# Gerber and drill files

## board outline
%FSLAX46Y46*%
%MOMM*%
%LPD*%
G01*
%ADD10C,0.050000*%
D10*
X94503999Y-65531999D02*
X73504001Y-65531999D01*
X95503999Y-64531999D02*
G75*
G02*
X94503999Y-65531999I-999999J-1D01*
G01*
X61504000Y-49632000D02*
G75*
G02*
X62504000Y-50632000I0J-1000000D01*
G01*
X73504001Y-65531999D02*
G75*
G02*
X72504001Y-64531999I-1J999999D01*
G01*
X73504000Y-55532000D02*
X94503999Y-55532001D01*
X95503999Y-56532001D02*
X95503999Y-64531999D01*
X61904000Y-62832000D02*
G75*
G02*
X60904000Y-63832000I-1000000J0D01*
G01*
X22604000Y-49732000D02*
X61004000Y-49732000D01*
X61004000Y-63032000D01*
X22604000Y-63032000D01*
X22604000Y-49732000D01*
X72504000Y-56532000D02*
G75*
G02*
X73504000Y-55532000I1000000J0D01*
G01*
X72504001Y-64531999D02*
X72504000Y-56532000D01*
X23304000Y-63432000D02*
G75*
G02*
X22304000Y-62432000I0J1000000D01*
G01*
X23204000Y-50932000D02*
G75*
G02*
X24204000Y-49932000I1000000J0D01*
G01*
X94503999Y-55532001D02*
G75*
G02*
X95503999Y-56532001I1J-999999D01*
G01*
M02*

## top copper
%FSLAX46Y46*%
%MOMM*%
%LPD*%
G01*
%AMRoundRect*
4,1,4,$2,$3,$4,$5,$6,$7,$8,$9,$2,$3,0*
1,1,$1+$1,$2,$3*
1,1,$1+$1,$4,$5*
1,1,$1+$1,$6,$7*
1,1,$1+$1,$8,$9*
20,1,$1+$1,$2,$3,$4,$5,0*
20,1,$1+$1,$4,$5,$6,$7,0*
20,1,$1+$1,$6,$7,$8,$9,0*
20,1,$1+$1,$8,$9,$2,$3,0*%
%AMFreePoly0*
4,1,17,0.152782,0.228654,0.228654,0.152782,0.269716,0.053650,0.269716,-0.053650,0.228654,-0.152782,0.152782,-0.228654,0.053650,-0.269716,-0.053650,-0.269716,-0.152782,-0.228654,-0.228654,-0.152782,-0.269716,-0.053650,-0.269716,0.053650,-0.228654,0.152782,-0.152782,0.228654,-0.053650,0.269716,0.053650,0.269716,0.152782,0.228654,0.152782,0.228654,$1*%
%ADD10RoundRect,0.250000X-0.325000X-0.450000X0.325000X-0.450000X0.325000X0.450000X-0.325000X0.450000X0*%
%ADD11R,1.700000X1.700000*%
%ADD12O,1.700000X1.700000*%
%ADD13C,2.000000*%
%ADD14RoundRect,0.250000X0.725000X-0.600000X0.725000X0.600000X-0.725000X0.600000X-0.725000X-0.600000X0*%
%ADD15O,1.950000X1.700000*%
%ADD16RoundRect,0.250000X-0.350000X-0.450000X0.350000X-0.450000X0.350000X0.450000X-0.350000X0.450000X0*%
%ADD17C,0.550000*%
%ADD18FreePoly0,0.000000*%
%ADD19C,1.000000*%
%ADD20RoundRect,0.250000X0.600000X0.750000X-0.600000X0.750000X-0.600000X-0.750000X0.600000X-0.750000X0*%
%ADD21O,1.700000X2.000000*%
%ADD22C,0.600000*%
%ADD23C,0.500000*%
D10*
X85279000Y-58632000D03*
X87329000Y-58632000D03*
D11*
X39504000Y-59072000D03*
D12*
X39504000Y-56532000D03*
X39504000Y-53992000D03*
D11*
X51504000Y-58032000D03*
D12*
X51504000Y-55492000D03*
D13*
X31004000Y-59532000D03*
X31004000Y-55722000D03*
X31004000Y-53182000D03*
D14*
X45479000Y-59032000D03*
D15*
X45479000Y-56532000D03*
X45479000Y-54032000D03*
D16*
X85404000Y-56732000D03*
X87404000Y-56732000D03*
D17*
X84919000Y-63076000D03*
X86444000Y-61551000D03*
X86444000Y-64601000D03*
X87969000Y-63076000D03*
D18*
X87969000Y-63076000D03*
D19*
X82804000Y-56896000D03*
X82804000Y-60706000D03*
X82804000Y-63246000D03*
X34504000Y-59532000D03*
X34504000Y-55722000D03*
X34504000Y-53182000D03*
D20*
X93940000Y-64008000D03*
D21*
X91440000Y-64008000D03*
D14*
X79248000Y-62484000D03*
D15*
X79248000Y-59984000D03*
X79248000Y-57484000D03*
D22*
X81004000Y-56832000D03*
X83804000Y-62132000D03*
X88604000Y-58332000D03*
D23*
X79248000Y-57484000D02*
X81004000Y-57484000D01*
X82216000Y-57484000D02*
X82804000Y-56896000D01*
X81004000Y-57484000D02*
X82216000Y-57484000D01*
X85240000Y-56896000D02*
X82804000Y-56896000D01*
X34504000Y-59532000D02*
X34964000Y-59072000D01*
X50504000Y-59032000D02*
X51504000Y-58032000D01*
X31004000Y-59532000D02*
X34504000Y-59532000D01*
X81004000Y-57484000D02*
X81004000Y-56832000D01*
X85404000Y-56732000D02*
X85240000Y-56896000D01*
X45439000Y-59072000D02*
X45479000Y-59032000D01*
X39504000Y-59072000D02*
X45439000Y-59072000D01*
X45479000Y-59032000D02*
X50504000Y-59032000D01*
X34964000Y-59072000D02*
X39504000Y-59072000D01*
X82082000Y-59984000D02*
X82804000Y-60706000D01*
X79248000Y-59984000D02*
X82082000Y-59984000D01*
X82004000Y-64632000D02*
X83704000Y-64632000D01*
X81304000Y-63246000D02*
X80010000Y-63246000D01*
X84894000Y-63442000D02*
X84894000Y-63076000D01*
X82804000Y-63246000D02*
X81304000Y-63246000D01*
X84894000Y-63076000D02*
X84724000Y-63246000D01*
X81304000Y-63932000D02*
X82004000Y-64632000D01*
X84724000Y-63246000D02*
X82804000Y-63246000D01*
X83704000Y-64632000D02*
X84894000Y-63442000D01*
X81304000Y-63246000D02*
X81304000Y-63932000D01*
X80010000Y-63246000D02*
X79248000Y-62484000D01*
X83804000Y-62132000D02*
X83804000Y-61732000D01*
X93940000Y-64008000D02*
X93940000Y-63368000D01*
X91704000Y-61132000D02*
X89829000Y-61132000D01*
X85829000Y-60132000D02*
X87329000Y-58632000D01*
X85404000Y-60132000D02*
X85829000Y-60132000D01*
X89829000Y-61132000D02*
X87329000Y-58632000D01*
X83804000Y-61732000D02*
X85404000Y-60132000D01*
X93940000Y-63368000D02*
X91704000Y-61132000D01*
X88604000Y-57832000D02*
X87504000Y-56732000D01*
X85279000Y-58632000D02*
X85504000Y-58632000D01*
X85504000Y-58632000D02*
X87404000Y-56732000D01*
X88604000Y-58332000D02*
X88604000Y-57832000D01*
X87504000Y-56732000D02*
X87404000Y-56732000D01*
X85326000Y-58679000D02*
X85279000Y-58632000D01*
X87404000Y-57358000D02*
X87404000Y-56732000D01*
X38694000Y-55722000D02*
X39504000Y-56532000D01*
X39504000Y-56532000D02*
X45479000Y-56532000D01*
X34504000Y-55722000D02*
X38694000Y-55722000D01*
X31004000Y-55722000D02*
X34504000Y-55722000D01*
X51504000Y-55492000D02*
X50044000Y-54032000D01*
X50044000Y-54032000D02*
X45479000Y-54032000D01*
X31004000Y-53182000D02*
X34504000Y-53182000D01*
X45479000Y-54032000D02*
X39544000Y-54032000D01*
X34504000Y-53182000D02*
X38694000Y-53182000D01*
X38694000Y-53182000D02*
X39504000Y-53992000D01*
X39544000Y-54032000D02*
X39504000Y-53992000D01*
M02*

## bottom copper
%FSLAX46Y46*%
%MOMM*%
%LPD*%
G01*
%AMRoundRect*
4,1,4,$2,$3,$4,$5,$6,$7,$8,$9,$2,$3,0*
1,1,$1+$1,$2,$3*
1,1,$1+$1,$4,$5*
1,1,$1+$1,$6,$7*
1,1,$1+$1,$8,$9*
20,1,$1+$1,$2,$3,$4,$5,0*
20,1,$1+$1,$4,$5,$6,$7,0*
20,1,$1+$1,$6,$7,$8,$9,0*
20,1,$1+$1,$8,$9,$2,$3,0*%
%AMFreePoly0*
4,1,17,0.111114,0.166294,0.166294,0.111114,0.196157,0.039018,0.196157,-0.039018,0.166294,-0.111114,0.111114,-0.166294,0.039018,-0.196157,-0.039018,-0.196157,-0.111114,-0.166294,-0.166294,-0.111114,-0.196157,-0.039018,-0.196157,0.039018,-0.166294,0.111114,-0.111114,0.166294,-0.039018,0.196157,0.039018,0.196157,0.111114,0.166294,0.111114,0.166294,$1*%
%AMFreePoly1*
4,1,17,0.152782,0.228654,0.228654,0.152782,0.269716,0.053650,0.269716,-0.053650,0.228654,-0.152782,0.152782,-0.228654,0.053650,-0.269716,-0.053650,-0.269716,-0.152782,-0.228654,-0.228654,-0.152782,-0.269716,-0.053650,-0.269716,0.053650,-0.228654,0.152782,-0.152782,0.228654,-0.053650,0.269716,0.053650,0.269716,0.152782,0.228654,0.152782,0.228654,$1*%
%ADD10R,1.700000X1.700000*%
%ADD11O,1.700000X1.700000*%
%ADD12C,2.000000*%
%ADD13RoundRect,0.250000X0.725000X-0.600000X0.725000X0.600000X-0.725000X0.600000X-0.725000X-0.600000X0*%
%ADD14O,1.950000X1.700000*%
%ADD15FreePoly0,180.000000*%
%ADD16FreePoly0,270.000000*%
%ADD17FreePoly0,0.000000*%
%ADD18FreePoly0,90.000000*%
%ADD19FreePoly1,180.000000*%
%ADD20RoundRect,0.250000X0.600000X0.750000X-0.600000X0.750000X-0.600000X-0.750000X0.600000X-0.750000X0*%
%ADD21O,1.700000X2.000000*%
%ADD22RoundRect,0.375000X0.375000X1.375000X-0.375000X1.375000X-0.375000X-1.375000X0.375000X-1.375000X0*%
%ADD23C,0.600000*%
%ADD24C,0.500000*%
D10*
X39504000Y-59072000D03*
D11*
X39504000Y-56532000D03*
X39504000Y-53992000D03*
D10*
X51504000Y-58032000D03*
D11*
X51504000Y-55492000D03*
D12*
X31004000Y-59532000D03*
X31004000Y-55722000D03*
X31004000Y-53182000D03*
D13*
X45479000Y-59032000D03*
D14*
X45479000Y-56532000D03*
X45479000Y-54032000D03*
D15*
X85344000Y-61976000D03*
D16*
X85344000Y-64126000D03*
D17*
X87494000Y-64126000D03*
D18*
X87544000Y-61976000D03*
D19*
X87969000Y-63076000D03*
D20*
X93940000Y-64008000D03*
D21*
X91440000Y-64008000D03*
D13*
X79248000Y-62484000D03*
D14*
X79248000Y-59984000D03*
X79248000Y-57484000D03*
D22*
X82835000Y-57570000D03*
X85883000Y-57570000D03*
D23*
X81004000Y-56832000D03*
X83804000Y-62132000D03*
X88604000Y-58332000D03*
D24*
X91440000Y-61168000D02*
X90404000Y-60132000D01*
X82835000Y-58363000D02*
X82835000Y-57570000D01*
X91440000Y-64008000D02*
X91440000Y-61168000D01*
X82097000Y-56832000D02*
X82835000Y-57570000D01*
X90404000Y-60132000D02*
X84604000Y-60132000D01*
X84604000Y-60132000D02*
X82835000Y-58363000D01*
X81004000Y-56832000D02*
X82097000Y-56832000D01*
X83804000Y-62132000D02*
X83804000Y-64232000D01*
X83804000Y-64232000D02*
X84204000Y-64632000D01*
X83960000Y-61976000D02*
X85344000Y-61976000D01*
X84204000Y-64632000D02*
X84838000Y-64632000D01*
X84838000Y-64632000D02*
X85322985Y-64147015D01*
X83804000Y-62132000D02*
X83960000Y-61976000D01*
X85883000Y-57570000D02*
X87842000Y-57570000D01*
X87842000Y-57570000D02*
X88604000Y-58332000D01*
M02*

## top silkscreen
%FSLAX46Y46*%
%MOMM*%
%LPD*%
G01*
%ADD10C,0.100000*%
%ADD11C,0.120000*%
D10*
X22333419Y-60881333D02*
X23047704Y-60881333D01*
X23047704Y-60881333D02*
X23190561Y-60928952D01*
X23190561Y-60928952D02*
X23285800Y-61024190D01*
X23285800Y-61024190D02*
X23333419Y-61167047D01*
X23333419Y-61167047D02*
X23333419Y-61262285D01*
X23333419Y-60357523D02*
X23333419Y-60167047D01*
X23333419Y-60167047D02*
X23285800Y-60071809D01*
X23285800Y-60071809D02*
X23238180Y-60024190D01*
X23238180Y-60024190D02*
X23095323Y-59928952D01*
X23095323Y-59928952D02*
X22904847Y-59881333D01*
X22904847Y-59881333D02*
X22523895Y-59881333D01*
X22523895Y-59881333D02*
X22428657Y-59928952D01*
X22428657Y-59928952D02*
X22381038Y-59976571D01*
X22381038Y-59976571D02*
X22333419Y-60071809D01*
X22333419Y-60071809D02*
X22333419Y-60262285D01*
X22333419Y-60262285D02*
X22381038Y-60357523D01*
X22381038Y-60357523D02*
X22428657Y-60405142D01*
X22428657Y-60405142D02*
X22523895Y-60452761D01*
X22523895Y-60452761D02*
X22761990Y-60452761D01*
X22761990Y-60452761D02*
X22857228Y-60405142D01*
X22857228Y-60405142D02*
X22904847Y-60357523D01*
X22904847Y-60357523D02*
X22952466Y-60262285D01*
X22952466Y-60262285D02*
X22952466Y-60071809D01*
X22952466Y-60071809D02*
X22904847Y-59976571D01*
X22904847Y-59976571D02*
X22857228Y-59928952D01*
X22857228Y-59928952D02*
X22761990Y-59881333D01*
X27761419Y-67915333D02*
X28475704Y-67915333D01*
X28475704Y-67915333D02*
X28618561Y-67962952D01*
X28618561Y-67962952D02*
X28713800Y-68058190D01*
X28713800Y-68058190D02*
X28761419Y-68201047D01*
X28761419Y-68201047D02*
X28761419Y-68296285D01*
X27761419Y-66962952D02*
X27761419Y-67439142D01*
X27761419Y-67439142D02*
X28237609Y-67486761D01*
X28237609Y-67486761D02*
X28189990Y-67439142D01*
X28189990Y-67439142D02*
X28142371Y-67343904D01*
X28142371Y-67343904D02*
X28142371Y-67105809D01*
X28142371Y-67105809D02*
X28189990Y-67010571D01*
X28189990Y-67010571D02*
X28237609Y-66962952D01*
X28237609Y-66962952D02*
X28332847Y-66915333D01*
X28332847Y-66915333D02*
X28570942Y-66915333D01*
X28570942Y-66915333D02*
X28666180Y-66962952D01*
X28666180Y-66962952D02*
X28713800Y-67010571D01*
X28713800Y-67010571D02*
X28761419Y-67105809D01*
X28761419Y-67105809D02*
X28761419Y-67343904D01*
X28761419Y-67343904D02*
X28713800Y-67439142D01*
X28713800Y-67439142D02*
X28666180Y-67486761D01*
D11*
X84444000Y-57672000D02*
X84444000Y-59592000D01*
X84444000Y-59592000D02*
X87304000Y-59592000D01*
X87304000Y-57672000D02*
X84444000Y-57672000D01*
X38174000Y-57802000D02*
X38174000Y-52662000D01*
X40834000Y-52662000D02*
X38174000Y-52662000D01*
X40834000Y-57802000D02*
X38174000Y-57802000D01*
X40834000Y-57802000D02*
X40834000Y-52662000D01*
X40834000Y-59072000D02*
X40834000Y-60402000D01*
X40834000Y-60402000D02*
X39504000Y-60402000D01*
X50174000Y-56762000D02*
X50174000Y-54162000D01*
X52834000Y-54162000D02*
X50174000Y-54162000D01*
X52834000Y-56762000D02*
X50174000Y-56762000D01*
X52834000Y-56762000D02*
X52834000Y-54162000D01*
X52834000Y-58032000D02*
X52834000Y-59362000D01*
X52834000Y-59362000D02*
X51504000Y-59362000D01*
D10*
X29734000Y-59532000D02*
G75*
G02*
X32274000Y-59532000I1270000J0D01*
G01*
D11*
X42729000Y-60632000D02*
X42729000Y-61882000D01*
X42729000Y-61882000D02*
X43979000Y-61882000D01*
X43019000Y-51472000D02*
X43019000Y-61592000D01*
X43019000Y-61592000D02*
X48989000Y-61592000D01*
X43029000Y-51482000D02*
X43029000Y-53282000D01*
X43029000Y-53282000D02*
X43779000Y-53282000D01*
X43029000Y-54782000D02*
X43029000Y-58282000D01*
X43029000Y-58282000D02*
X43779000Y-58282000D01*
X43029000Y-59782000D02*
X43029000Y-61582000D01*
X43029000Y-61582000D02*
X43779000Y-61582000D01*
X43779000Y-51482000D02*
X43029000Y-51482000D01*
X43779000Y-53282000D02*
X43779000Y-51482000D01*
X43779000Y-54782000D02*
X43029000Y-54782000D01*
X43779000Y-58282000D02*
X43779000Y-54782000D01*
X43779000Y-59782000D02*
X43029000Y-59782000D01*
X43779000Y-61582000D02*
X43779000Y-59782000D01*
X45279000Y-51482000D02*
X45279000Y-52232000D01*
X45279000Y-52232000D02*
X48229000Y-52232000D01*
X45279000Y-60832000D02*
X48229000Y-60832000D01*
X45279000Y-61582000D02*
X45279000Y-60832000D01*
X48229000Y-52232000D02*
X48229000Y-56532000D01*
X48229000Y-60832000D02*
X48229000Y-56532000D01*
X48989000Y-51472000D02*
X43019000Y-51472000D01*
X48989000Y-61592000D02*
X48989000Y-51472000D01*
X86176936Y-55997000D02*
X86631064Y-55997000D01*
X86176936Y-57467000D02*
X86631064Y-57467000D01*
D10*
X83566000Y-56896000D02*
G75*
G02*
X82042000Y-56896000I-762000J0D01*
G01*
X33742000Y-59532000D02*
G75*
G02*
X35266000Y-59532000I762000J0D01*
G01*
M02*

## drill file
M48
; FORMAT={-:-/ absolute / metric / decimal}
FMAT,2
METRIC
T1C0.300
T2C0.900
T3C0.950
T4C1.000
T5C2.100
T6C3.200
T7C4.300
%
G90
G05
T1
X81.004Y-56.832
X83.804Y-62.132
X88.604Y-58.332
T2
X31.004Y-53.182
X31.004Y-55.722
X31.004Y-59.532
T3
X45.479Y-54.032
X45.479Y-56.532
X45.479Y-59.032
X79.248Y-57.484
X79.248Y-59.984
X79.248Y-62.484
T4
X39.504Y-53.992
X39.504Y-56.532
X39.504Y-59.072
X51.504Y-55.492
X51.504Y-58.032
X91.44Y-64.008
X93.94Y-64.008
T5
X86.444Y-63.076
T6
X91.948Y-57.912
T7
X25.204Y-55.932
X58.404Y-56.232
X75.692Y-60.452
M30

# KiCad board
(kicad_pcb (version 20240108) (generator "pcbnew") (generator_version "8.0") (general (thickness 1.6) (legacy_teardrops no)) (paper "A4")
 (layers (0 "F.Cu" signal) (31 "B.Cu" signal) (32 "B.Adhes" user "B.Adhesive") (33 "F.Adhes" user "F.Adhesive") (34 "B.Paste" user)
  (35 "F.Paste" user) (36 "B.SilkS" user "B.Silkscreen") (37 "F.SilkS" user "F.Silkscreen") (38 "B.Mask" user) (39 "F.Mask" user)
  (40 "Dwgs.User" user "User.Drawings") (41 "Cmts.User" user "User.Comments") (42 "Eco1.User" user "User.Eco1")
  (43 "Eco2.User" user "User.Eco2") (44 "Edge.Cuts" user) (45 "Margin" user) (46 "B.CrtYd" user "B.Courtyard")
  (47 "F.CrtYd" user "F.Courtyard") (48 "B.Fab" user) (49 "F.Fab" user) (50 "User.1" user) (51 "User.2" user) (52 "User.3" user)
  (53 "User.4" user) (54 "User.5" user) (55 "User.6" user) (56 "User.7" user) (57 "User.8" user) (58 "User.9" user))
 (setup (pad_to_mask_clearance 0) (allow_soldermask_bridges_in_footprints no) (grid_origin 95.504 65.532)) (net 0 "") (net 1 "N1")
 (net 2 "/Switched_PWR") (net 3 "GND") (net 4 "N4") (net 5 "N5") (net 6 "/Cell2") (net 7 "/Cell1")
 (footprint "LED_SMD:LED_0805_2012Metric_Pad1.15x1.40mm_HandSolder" (layer "F.Cu") (at 86.304 58.632)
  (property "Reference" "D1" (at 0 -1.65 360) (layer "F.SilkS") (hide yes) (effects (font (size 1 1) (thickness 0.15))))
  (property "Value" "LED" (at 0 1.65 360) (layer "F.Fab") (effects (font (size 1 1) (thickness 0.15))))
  (fp_line (start -1.86 -0.96) (end -1.86 0.96) (stroke (width 0.12) (type solid)) (layer "F.SilkS"))
  (fp_line (start -1.86 0.96) (end 1 0.96) (stroke (width 0.12) (type solid)) (layer "F.SilkS"))
  (fp_line (start 1 -0.96) (end -1.86 -0.96) (stroke (width 0.12) (type solid)) (layer "F.SilkS"))
  (pad "1" smd roundrect (at -1.025 0) (size 1.15 1.4) (layers "F.Cu" "F.Paste" "F.Mask") (roundrect_rratio 0.217391) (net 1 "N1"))
  (pad "2" smd roundrect (at 1.025 0) (size 1.15 1.4) (layers "F.Cu" "F.Paste" "F.Mask") (roundrect_rratio 0.217391) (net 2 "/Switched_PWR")))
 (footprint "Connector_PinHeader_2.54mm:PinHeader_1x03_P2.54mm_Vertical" (layer "F.Cu") (at 39.504 59.072 180)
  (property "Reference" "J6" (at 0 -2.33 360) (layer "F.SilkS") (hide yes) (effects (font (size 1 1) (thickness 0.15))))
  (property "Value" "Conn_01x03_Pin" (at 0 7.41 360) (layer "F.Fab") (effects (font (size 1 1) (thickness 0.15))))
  (fp_line (start 1.33 1.27) (end 1.33 6.41) (stroke (width 0.12) (type solid)) (layer "F.SilkS"))
  (fp_line (start -1.33 6.41) (end 1.33 6.41) (stroke (width 0.12) (type solid)) (layer "F.SilkS"))
  (fp_line (start -1.33 1.27) (end 1.33 1.27) (stroke (width 0.12) (type solid)) (layer "F.SilkS"))
  (fp_line (start -1.33 1.27) (end -1.33 6.41) (stroke (width 0.12) (type solid)) (layer "F.SilkS"))
  (fp_line (start -1.33 0) (end -1.33 -1.33) (stroke (width 0.12) (type solid)) (layer "F.SilkS"))
  (fp_line (start -1.33 -1.33) (end 0 -1.33) (stroke (width 0.12) (type solid)) (layer "F.SilkS"))
  (pad "1" thru_hole rect (at 0 0 180) (size 1.7 1.7) (drill 1) (layers "*.Cu" "*.Mask") (remove_unused_layers no) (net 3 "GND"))
  (pad "2" thru_hole oval (at 0 2.54 180) (size 1.7 1.7) (drill 1) (layers "*.Cu" "*.Mask") (remove_unused_layers no) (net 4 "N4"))
  (pad "3" thru_hole oval (at 0 5.08 180) (size 1.7 1.7) (drill 1) (layers "*.Cu" "*.Mask") (remove_unused_layers no) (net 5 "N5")))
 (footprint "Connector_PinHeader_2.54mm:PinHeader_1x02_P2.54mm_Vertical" (layer "F.Cu") (at 51.504 58.032 180)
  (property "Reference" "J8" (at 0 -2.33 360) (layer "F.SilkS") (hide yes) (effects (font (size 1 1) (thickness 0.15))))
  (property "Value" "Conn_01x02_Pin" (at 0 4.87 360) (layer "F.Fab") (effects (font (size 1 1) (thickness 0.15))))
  (fp_line (start 1.33 1.27) (end 1.33 3.87) (stroke (width 0.12) (type solid)) (layer "F.SilkS"))
  (fp_line (start -1.33 3.87) (end 1.33 3.87) (stroke (width 0.12) (type solid)) (layer "F.SilkS"))
  (fp_line (start -1.33 1.27) (end 1.33 1.27) (stroke (width 0.12) (type solid)) (layer "F.SilkS"))
  (fp_line (start -1.33 1.27) (end -1.33 3.87) (stroke (width 0.12) (type solid)) (layer "F.SilkS"))
  (fp_line (start -1.33 0) (end -1.33 -1.33) (stroke (width 0.12) (type solid)) (layer "F.SilkS"))
  (fp_line (start -1.33 -1.33) (end 0 -1.33) (stroke (width 0.12) (type solid)) (layer "F.SilkS"))
  (pad "1" thru_hole rect (at 0 0 180) (size 1.7 1.7) (drill 1) (layers "*.Cu" "*.Mask") (remove_unused_layers no) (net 3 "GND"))
  (pad "2" thru_hole oval (at 0 2.54 180) (size 1.7 1.7) (drill 1) (layers "*.Cu" "*.Mask") (remove_unused_layers no) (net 5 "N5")))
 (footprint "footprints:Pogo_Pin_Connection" (layer "F.Cu") (at 31.004 59.532 90)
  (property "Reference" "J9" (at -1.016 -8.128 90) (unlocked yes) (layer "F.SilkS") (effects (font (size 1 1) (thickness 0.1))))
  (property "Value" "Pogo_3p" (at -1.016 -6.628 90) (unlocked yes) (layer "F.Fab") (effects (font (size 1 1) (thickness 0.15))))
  (fp_arc (start 0 -1.27) (mid 1.27 0) (end 0 1.27) (stroke (width 0.1) (type default)) (layer "F.SilkS"))
  (pad "1" thru_hole circle (at 0 0 270) (size 2 2) (drill 0.9) (layers "*.Cu" "*.Mask") (remove_unused_layers no) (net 3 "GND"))
  (pad "2" thru_hole circle (at 3.81 0 270) (size 2 2) (drill 0.9) (layers "*.Cu" "*.Mask") (remove_unused_layers no) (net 4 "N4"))
  (pad "3" thru_hole circle (at 6.35 0 270) (size 2 2) (drill 0.9) (layers "*.Cu" "*.Mask") (remove_unused_layers no) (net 5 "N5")))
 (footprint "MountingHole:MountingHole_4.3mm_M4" (layer "F.Cu") (at 25.204 55.932)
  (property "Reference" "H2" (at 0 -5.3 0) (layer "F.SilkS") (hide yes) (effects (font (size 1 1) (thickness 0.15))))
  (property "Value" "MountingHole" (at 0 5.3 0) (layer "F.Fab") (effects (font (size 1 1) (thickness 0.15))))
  (pad "" np_thru_hole circle (at 0 0) (size 4.3 4.3) (drill 4.3) (layers "*.Cu" "*.Mask")))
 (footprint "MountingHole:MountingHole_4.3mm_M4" (layer "F.Cu") (at 75.692 60.452)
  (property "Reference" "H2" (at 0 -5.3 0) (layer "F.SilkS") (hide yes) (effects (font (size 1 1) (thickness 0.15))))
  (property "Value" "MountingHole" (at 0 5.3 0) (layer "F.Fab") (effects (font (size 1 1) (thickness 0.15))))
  (pad "" np_thru_hole circle (at 0 0) (size 4.3 4.3) (drill 4.3) (layers "*.Cu" "*.Mask")))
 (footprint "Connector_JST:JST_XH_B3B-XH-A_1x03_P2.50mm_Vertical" (layer "F.Cu") (at 45.479 59.032 90)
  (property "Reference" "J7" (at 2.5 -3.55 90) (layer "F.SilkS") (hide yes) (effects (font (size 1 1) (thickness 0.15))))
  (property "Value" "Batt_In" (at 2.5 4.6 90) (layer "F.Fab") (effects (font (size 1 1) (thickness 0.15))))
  (fp_line (start -1.6 -2.75) (end -2.85 -2.75) (stroke (width 0.12) (type solid)) (layer "F.SilkS"))
  (fp_line (start -2.85 -2.75) (end -2.85 -1.5) (stroke (width 0.12) (type solid)) (layer "F.SilkS"))
  (fp_line (start 7.56 -2.46) (end -2.56 -2.46) (stroke (width 0.12) (type solid)) (layer "F.SilkS"))
  (fp_line (start -2.56 -2.46) (end -2.56 3.51) (stroke (width 0.12) (type solid)) (layer "F.SilkS"))
  (fp_line (start 7.55 -2.45) (end 5.75 -2.45) (stroke (width 0.12) (type solid)) (layer "F.SilkS"))
  (fp_line (start 5.75 -2.45) (end 5.75 -1.7) (stroke (width 0.12) (type solid)) (layer "F.SilkS"))
  (fp_line (start 4.25 -2.45) (end 0.75 -2.45) (stroke (width 0.12) (type solid)) (layer "F.SilkS"))
  (fp_line (start 0.75 -2.45) (end 0.75 -1.7) (stroke (width 0.12) (type solid)) (layer "F.SilkS"))
  (fp_line (start -0.75 -2.45) (end -2.55 -2.45) (stroke (width 0.12) (type solid)) (layer "F.SilkS"))
  (fp_line (start -2.55 -2.45) (end -2.55 -1.7) (stroke (width 0.12) (type solid)) (layer "F.SilkS"))
  (fp_line (start 7.55 -1.7) (end 7.55 -2.45) (stroke (width 0.12) (type solid)) (layer "F.SilkS"))
  (fp_line (start 5.75 -1.7) (end 7.55 -1.7) (stroke (width 0.12) (type solid)) (layer "F.SilkS"))
  (fp_line (start 4.25 -1.7) (end 4.25 -2.45) (stroke (width 0.12) (type solid)) (layer "F.SilkS"))
  (fp_line (start 0.75 -1.7) (end 4.25 -1.7) (stroke (width 0.12) (type solid)) (layer "F.SilkS"))
  (fp_line (start -0.75 -1.7) (end -0.75 -2.45) (stroke (width 0.12) (type solid)) (layer "F.SilkS"))
  (fp_line (start -2.55 -1.7) (end -0.75 -1.7) (stroke (width 0.12) (type solid)) (layer "F.SilkS"))
  (fp_line (start 7.55 -0.2) (end 6.8 -0.2) (stroke (width 0.12) (type solid)) (layer "F.SilkS"))
  (fp_line (start 6.8 -0.2) (end 6.8 2.75) (stroke (width 0.12) (type solid)) (layer "F.SilkS"))
  (fp_line (start -1.8 -0.2) (end -1.8 2.75) (stroke (width 0.12) (type solid)) (layer "F.SilkS"))
  (fp_line (start -2.55 -0.2) (end -1.8 -0.2) (stroke (width 0.12) (type solid)) (layer "F.SilkS"))
  (fp_line (start 6.8 2.75) (end 2.5 2.75) (stroke (width 0.12) (type solid)) (layer "F.SilkS"))
  (fp_line (start -1.8 2.75) (end 2.5 2.75) (stroke (width 0.12) (type solid)) (layer "F.SilkS"))
  (fp_line (start 7.56 3.51) (end 7.56 -2.46) (stroke (width 0.12) (type solid)) (layer "F.SilkS"))
  (fp_line (start -2.56 3.51) (end 7.56 3.51) (stroke (width 0.12) (type solid)) (layer "F.SilkS"))
  (pad "1" thru_hole roundrect (at 0 0 90) (size 1.7 1.95) (drill 0.95) (layers "*.Cu" "*.Mask") (remove_unused_layers no)
   (roundrect_rratio 0.147059) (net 3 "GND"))
  (pad "2" thru_hole oval (at 2.5 0 90) (size 1.7 1.95) (drill 0.95) (layers "*.Cu" "*.Mask") (remove_unused_layers no) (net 4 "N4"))
  (pad "3" thru_hole oval (at 5 0 90) (size 1.7 1.95) (drill 0.95) (layers "*.Cu" "*.Mask") (remove_unused_layers no) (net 5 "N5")))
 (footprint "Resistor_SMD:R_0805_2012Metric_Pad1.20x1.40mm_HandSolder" (layer "F.Cu") (at 86.404 56.732)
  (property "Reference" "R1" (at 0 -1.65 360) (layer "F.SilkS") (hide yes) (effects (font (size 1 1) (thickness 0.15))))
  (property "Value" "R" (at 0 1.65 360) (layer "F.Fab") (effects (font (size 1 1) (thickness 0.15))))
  (fp_line (start -0.227064 -0.735) (end 0.227064 -0.735) (stroke (width 0.12) (type solid)) (layer "F.SilkS"))
  (fp_line (start -0.227064 0.735) (end 0.227064 0.735) (stroke (width 0.12) (type solid)) (layer "F.SilkS"))
  (pad "1" smd roundrect (at -1 0) (size 1.2 1.4) (layers "F.Cu" "F.Paste" "F.Mask") (roundrect_rratio 0.208333) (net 3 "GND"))
  (pad "2" smd roundrect (at 1 0) (size 1.2 1.4) (layers "F.Cu" "F.Paste" "F.Mask") (roundrect_rratio 0.208333) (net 1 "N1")))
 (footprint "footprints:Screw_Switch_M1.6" (layer "F.Cu") (at 86.444 63.076)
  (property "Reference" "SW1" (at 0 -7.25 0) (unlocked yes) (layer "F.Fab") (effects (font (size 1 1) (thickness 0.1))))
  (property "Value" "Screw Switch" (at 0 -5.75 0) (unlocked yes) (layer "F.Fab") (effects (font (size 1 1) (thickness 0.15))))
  (pad "" smd custom (at -1.06066 -1.06066 180) (size 0.4 0.4) (layers "F.Paste") (thermal_bridge_angle 90)
   (options (clearance outline) (anchor circle)) (primitives))
  (pad "" smd custom (at -1.06066 1.06066 270) (size 0.4 0.4) (layers "F.Paste") (thermal_bridge_angle 90)
   (options (clearance outline) (anchor circle)) (primitives))
  (pad "" np_thru_hole circle (at 0 0) (size 2.1 2.1) (drill 2.1) (layers "F&B.Cu" "*.Mask"))
  (pad "" smd custom (at 1.06066 -1.06066 90) (size 0.4 0.4) (layers "F.Paste") (thermal_bridge_angle 90)
   (options (clearance outline) (anchor circle)) (primitives))
  (pad "" smd custom (at 1.06066 1.06066) (size 0.4 0.4) (layers "F.Paste") (thermal_bridge_angle 90)
   (options (clearance outline) (anchor circle)) (primitives))
  (pad "1" smd circle (at -1.525 0) (size 0.55 0.55) (layers "F.Cu") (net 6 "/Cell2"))
  (pad "1" smd circle (at 0 -1.525) (size 0.55 0.55) (layers "F.Cu") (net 6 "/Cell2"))
  (pad "1" smd circle (at 0 1.525) (size 0.55 0.55) (layers "F.Cu") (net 6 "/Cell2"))
  (pad "1" smd circle (at 1.525 0) (size 0.55 0.55) (layers "F.Cu") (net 6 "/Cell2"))
  (pad "1" smd custom (at 1.525 0) (size 0.55 0.55) (layers "F.Cu" "F.Mask") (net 6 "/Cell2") (thermal_bridge_angle 90)
   (options (clearance outline) (anchor circle)) (primitives))
  (pad "2" smd custom (at -1.1 -1.1 180) (size 0.4 0.4) (layers "B.Cu" "B.Paste" "B.Mask") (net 2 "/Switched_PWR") (thermal_bridge_angle 90)
   (options (clearance outline) (anchor circle)) (primitives))
  (pad "2" smd custom (at -1.1 1.05 270) (size 0.4 0.4) (layers "B.Cu" "B.Paste" "B.Mask") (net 2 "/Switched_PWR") (thermal_bridge_angle 90)
   (options (clearance outline) (anchor circle)) (primitives))
  (pad "2" smd custom (at 1.05 1.05) (size 0.4 0.4) (layers "B.Cu" "B.Paste" "B.Mask") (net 2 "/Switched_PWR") (thermal_bridge_angle 90)
   (options (clearance outline) (anchor circle)) (primitives))
  (pad "2" smd custom (at 1.1 -1.1 90) (size 0.4 0.4) (layers "B.Cu" "B.Paste" "B.Mask") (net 2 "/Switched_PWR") (thermal_bridge_angle 90)
   (options (clearance outline) (anchor circle)) (primitives))
  (pad "2" smd custom (at 1.525 0 180) (size 0.55 0.55) (layers "B.Cu") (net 2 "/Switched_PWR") (thermal_bridge_angle 90)
   (options (clearance outline) (anchor circle)) (primitives)))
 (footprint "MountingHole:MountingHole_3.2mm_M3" (layer "F.Cu") (at 91.948 57.912)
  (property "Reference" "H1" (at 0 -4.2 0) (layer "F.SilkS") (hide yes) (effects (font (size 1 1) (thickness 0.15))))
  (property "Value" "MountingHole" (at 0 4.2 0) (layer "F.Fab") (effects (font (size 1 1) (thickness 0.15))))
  (pad "" np_thru_hole circle (at 0 0) (size 3.2 3.2) (drill 3.2) (layers "*.Cu" "*.Mask")))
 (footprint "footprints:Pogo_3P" (layer "F.Cu") (at 82.804 56.896 -90)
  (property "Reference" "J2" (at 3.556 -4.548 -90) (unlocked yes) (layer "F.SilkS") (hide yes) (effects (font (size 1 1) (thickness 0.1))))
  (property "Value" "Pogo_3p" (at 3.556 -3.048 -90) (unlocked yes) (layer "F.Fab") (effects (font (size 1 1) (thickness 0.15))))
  (fp_arc (start 0 -0.762) (mid 0.762 0) (end 0 0.762) (stroke (width 0.1) (type default)) (layer "F.SilkS"))
  (pad "1" smd circle (at 0 0 90) (size 1 1) (layers "F.Cu" "F.Mask") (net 3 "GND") (thermal_bridge_angle 90))
  (pad "2" smd circle (at 3.81 0 90) (size 1 1) (layers "F.Cu" "F.Mask") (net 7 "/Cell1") (thermal_bridge_angle 90))
  (pad "3" smd circle (at 6.35 0 90) (size 1 1) (layers "F.Cu" "F.Mask") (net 6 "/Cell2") (thermal_bridge_angle 90)))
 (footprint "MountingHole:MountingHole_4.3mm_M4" (layer "F.Cu") (at 58.404 56.232)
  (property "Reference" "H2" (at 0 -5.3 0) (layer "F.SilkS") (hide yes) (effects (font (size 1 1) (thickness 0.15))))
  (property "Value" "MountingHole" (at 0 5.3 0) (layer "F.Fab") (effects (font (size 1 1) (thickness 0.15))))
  (pad "" np_thru_hole circle (at 0 0) (size 4.3 4.3) (drill 4.3) (layers "*.Cu" "*.Mask")))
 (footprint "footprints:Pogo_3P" (layer "F.Cu") (at 34.504 59.532 90)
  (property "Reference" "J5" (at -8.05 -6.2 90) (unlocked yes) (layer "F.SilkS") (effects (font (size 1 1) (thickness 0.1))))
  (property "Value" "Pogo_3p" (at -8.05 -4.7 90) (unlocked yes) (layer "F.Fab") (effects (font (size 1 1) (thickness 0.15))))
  (fp_arc (start 0 -0.762) (mid 0.762 0) (end 0 0.762) (stroke (width 0.1) (type default)) (layer "F.SilkS"))
  (pad "1" smd circle (at 0 0 270) (size 1 1) (layers "F.Cu" "F.Mask") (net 3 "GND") (thermal_bridge_angle 90))
  (pad "2" smd circle (at 3.81 0 270) (size 1 1) (layers "F.Cu" "F.Mask") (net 4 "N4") (thermal_bridge_angle 90))
  (pad "3" smd circle (at 6.35 0 270) (size 1 1) (layers "F.Cu" "F.Mask") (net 5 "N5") (thermal_bridge_angle 90)))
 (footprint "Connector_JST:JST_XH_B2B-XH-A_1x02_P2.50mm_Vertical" (layer "B.Cu") (at 93.94 64.008 180)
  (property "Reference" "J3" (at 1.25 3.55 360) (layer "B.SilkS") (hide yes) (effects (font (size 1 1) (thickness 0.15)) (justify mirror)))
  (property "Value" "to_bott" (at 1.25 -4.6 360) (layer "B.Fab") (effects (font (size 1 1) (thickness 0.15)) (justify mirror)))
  (pad "1" thru_hole roundrect (at 0 0 180) (size 1.7 2) (drill 1) (layers "*.Cu" "*.Mask") (remove_unused_layers no)
   (roundrect_rratio 0.147059) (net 2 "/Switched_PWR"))
  (pad "2" thru_hole oval (at 2.5 0 180) (size 1.7 2) (drill 1) (layers "*.Cu" "*.Mask") (remove_unused_layers no) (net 3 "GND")))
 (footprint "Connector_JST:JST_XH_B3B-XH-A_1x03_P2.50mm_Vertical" (layer "B.Cu") (at 79.248 62.484 90)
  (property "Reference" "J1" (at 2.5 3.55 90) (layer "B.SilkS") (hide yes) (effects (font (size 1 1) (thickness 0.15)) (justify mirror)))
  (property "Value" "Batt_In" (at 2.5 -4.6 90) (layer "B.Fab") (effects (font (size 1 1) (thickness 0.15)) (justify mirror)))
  (pad "1" thru_hole roundrect (at 0 0 90) (size 1.7 1.95) (drill 0.95) (layers "*.Cu" "*.Mask") (remove_unused_layers no)
   (roundrect_rratio 0.147059) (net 6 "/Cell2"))
  (pad "2" thru_hole oval (at 2.5 0 90) (size 1.7 1.95) (drill 0.95) (layers "*.Cu" "*.Mask") (remove_unused_layers no) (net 7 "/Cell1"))
  (pad "3" thru_hole oval (at 5 0 90) (size 1.7 1.95) (drill 0.95) (layers "*.Cu" "*.Mask") (remove_unused_layers no) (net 3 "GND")))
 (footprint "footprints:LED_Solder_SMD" (layer "B.Cu") (at 82.835 57.57)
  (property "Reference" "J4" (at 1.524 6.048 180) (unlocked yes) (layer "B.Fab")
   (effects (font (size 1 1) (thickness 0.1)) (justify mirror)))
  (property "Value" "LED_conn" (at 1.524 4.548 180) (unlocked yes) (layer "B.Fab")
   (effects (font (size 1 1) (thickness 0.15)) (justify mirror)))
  (pad "1" smd roundrect (at 0 0 180) (size 1.5 3.5) (layers "B.Cu" "B.Mask") (roundrect_rratio 0.25) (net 3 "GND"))
  (pad "2" smd roundrect (at 3.048 0 180) (size 1.5 3.5) (layers "B.Cu" "B.Mask") (roundrect_rratio 0.25) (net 1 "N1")))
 (gr_line (start 94.503999 65.531999) (end 73.504001 65.531999) (stroke (width 0.05) (type default)) (layer "Edge.Cuts"))
 (gr_arc (start 95.503999 64.531999) (mid 95.211106 65.239106) (end 94.503999 65.531999) (stroke (width 0.05) (type default))
  (layer "Edge.Cuts"))
 (gr_arc (start 61.504 49.632) (mid 62.211107 49.924893) (end 62.504 50.632) (stroke (width 0.05) (type default)) (layer "Edge.Cuts"))
 (gr_arc (start 73.504001 65.531999) (mid 72.796894 65.239106) (end 72.504001 64.531999) (stroke (width 0.05) (type default))
  (layer "Edge.Cuts"))
 (gr_line (start 73.504 55.532) (end 94.503999 55.532001) (stroke (width 0.05) (type default)) (layer "Edge.Cuts"))
 (gr_line (start 95.503999 56.532001) (end 95.503999 64.531999) (stroke (width 0.05) (type default)) (layer "Edge.Cuts"))
 (gr_arc (start 61.904 62.832) (mid 61.611107 63.539107) (end 60.904 63.832) (stroke (width 0.05) (type default)) (layer "Edge.Cuts"))
 (gr_rect (start 22.604 49.732) (end 61.004 63.032) (stroke (width 0.05) (type default)) (fill none) (layer "Edge.Cuts"))
 (gr_arc (start 72.504 56.532) (mid 72.796893 55.824893) (end 73.504 55.532) (stroke (width 0.05) (type default)) (layer "Edge.Cuts"))
 (gr_line (start 72.504001 64.531999) (end 72.504 56.532) (stroke (width 0.05) (type default)) (layer "Edge.Cuts"))
 (gr_arc (start 23.304 63.432) (mid 22.596893 63.139107) (end 22.304 62.432) (stroke (width 0.05) (type default)) (layer "Edge.Cuts"))
 (gr_arc (start 23.204 50.932) (mid 23.496893 50.224893) (end 24.204 49.932) (stroke (width 0.05) (type default)) (layer "Edge.Cuts"))
 (gr_arc (start 94.503999 55.532001) (mid 95.211106 55.824894) (end 95.503999 56.532001) (stroke (width 0.05) (type default))
  (layer "Edge.Cuts"))
 (segment (start 79.248 57.484) (end 81.004 57.484) (width 0.5) (layer "F.Cu") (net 3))
 (segment (start 82.216 57.484) (end 82.804 56.896) (width 0.5) (layer "F.Cu") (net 3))
 (segment (start 81.004 57.484) (end 82.216 57.484) (width 0.5) (layer "F.Cu") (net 3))
 (segment (start 85.24 56.896) (end 82.804 56.896) (width 0.5) (layer "F.Cu") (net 3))
 (segment (start 34.504 59.532) (end 34.964 59.072) (width 0.5) (layer "F.Cu") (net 3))
 (segment (start 50.504 59.032) (end 51.504 58.032) (width 0.5) (layer "F.Cu") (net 3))
 (segment (start 31.004 59.532) (end 34.504 59.532) (width 0.5) (layer "F.Cu") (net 3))
 (segment (start 81.004 57.484) (end 81.004 56.832) (width 0.5) (layer "F.Cu") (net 3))
 (segment (start 85.404 56.732) (end 85.24 56.896) (width 0.5) (layer "F.Cu") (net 3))
 (segment (start 45.439 59.072) (end 45.479 59.032) (width 0.5) (layer "F.Cu") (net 3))
 (segment (start 39.504 59.072) (end 45.439 59.072) (width 0.5) (layer "F.Cu") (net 3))
 (segment (start 45.479 59.032) (end 50.504 59.032) (width 0.5) (layer "F.Cu") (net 3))
 (segment (start 34.964 59.072) (end 39.504 59.072) (width 0.5) (layer "F.Cu") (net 3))
 (via (at 81.004 56.832) (size 0.6) (drill 0.3) (layers "F.Cu" "B.Cu") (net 3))
 (segment (start 91.44 61.168) (end 90.404 60.132) (width 0.5) (layer "B.Cu") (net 3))
 (segment (start 82.835 58.363) (end 82.835 57.57) (width 0.5) (layer "B.Cu") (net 3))
 (segment (start 91.44 64.008) (end 91.44 61.168) (width 0.5) (layer "B.Cu") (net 3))
 (segment (start 82.097 56.832) (end 82.835 57.57) (width 0.5) (layer "B.Cu") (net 3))
 (segment (start 90.404 60.132) (end 84.604 60.132) (width 0.5) (layer "B.Cu") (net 3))
 (segment (start 84.604 60.132) (end 82.835 58.363) (width 0.5) (layer "B.Cu") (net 3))
 (segment (start 81.004 56.832) (end 82.097 56.832) (width 0.5) (layer "B.Cu") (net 3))
 (segment (start 82.082 59.984) (end 82.804 60.706) (width 0.5) (layer "F.Cu") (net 7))
 (segment (start 79.248 59.984) (end 82.082 59.984) (width 0.5) (layer "F.Cu") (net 7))
 (segment (start 82.004 64.632) (end 83.704 64.632) (width 0.5) (layer "F.Cu") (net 6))
 (segment (start 81.304 63.246) (end 80.01 63.246) (width 0.5) (layer "F.Cu") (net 6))
 (segment (start 84.894 63.442) (end 84.894 63.076) (width 0.5) (layer "F.Cu") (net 6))
 (segment (start 82.804 63.246) (end 81.304 63.246) (width 0.5) (layer "F.Cu") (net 6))
 (segment (start 84.894 63.076) (end 84.724 63.246) (width 0.5) (layer "F.Cu") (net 6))
 (segment (start 81.304 63.932) (end 82.004 64.632) (width 0.5) (layer "F.Cu") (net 6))
 (segment (start 84.724 63.246) (end 82.804 63.246) (width 0.5) (layer "F.Cu") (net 6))
 (segment (start 83.704 64.632) (end 84.894 63.442) (width 0.5) (layer "F.Cu") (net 6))
 (segment (start 81.304 63.246) (end 81.304 63.932) (width 0.5) (layer "F.Cu") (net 6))
 (segment (start 80.01 63.246) (end 79.248 62.484) (width 0.5) (layer "F.Cu") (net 6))
 (segment (start 83.804 62.132) (end 83.804 61.732) (width 0.5) (layer "F.Cu") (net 2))
 (segment (start 93.94 64.008) (end 93.94 63.368) (width 0.5) (layer "F.Cu") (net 2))
 (segment (start 91.704 61.132) (end 89.829 61.132) (width 0.5) (layer "F.Cu") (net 2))
 (segment (start 85.829 60.132) (end 87.329 58.632) (width 0.5) (layer "F.Cu") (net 2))
 (segment (start 85.404 60.132) (end 85.829 60.132) (width 0.5) (layer "F.Cu") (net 2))
 (segment (start 89.829 61.132) (end 87.329 58.632) (width 0.5) (layer "F.Cu") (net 2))
 (segment (start 83.804 61.732) (end 85.404 60.132) (width 0.5) (layer "F.Cu") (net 2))
 (segment (start 93.94 63.368) (end 91.704 61.132) (width 0.5) (layer "F.Cu") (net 2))
 (via (at 83.804 62.132) (size 0.6) (drill 0.3) (layers "F.Cu" "B.Cu") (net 2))
 (segment (start 83.804 62.132) (end 83.804 64.232) (width 0.5) (layer "B.Cu") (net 2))
 (segment (start 83.804 64.232) (end 84.204 64.632) (width 0.5) (layer "B.Cu") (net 2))
 (segment (start 83.96 61.976) (end 85.344 61.976) (width 0.5) (layer "B.Cu") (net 2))
 (segment (start 84.204 64.632) (end 84.838 64.632) (width 0.5) (layer "B.Cu") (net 2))
 (segment (start 84.838 64.632) (end 85.322985 64.147015) (width 0.5) (layer "B.Cu") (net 2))
 (segment (start 83.804 62.132) (end 83.96 61.976) (width 0.5) (layer "B.Cu") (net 2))
 (segment (start 88.604 57.832) (end 87.504 56.732) (width 0.5) (layer "F.Cu") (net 1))
 (segment (start 85.279 58.632) (end 85.504 58.632) (width 0.5) (layer "F.Cu") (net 1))
 (segment (start 85.504 58.632) (end 87.404 56.732) (width 0.5) (layer "F.Cu") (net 1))
 (segment (start 88.604 58.332) (end 88.604 57.832) (width 0.5) (layer "F.Cu") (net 1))
 (segment (start 87.504 56.732) (end 87.404 56.732) (width 0.5) (layer "F.Cu") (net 1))
 (segment (start 85.326 58.679) (end 85.279 58.632) (width 0.5) (layer "F.Cu") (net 1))
 (segment (start 87.404 57.358) (end 87.404 56.732) (width 0.5) (layer "F.Cu") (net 1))
 (via (at 88.604 58.332) (size 0.6) (drill 0.3) (layers "F.Cu" "B.Cu") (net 1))
 (segment (start 85.883 57.57) (end 87.842 57.57) (width 0.5) (layer "B.Cu") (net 1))
 (segment (start 87.842 57.57) (end 88.604 58.332) (width 0.5) (layer "B.Cu") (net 1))
 (segment (start 38.694 55.722) (end 39.504 56.532) (width 0.5) (layer "F.Cu") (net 4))
 (segment (start 39.504 56.532) (end 45.479 56.532) (width 0.5) (layer "F.Cu") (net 4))
 (segment (start 34.504 55.722) (end 38.694 55.722) (width 0.5) (layer "F.Cu") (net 4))
 (segment (start 31.004 55.722) (end 34.504 55.722) (width 0.5) (layer "F.Cu") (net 4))
 (segment (start 51.504 55.492) (end 50.044 54.032) (width 0.5) (layer "F.Cu") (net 5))
 (segment (start 50.044 54.032) (end 45.479 54.032) (width 0.5) (layer "F.Cu") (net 5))
 (segment (start 31.004 53.182) (end 34.504 53.182) (width 0.5) (layer "F.Cu") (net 5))
 (segment (start 45.479 54.032) (end 39.544 54.032) (width 0.5) (layer "F.Cu") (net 5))
 (segment (start 34.504 53.182) (end 38.694 53.182) (width 0.5) (layer "F.Cu") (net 5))
 (segment (start 38.694 53.182) (end 39.504 53.992) (width 0.5) (layer "F.Cu") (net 5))
 (segment (start 39.544 54.032) (end 39.504 53.992) (width 0.5) (layer "F.Cu") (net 5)))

